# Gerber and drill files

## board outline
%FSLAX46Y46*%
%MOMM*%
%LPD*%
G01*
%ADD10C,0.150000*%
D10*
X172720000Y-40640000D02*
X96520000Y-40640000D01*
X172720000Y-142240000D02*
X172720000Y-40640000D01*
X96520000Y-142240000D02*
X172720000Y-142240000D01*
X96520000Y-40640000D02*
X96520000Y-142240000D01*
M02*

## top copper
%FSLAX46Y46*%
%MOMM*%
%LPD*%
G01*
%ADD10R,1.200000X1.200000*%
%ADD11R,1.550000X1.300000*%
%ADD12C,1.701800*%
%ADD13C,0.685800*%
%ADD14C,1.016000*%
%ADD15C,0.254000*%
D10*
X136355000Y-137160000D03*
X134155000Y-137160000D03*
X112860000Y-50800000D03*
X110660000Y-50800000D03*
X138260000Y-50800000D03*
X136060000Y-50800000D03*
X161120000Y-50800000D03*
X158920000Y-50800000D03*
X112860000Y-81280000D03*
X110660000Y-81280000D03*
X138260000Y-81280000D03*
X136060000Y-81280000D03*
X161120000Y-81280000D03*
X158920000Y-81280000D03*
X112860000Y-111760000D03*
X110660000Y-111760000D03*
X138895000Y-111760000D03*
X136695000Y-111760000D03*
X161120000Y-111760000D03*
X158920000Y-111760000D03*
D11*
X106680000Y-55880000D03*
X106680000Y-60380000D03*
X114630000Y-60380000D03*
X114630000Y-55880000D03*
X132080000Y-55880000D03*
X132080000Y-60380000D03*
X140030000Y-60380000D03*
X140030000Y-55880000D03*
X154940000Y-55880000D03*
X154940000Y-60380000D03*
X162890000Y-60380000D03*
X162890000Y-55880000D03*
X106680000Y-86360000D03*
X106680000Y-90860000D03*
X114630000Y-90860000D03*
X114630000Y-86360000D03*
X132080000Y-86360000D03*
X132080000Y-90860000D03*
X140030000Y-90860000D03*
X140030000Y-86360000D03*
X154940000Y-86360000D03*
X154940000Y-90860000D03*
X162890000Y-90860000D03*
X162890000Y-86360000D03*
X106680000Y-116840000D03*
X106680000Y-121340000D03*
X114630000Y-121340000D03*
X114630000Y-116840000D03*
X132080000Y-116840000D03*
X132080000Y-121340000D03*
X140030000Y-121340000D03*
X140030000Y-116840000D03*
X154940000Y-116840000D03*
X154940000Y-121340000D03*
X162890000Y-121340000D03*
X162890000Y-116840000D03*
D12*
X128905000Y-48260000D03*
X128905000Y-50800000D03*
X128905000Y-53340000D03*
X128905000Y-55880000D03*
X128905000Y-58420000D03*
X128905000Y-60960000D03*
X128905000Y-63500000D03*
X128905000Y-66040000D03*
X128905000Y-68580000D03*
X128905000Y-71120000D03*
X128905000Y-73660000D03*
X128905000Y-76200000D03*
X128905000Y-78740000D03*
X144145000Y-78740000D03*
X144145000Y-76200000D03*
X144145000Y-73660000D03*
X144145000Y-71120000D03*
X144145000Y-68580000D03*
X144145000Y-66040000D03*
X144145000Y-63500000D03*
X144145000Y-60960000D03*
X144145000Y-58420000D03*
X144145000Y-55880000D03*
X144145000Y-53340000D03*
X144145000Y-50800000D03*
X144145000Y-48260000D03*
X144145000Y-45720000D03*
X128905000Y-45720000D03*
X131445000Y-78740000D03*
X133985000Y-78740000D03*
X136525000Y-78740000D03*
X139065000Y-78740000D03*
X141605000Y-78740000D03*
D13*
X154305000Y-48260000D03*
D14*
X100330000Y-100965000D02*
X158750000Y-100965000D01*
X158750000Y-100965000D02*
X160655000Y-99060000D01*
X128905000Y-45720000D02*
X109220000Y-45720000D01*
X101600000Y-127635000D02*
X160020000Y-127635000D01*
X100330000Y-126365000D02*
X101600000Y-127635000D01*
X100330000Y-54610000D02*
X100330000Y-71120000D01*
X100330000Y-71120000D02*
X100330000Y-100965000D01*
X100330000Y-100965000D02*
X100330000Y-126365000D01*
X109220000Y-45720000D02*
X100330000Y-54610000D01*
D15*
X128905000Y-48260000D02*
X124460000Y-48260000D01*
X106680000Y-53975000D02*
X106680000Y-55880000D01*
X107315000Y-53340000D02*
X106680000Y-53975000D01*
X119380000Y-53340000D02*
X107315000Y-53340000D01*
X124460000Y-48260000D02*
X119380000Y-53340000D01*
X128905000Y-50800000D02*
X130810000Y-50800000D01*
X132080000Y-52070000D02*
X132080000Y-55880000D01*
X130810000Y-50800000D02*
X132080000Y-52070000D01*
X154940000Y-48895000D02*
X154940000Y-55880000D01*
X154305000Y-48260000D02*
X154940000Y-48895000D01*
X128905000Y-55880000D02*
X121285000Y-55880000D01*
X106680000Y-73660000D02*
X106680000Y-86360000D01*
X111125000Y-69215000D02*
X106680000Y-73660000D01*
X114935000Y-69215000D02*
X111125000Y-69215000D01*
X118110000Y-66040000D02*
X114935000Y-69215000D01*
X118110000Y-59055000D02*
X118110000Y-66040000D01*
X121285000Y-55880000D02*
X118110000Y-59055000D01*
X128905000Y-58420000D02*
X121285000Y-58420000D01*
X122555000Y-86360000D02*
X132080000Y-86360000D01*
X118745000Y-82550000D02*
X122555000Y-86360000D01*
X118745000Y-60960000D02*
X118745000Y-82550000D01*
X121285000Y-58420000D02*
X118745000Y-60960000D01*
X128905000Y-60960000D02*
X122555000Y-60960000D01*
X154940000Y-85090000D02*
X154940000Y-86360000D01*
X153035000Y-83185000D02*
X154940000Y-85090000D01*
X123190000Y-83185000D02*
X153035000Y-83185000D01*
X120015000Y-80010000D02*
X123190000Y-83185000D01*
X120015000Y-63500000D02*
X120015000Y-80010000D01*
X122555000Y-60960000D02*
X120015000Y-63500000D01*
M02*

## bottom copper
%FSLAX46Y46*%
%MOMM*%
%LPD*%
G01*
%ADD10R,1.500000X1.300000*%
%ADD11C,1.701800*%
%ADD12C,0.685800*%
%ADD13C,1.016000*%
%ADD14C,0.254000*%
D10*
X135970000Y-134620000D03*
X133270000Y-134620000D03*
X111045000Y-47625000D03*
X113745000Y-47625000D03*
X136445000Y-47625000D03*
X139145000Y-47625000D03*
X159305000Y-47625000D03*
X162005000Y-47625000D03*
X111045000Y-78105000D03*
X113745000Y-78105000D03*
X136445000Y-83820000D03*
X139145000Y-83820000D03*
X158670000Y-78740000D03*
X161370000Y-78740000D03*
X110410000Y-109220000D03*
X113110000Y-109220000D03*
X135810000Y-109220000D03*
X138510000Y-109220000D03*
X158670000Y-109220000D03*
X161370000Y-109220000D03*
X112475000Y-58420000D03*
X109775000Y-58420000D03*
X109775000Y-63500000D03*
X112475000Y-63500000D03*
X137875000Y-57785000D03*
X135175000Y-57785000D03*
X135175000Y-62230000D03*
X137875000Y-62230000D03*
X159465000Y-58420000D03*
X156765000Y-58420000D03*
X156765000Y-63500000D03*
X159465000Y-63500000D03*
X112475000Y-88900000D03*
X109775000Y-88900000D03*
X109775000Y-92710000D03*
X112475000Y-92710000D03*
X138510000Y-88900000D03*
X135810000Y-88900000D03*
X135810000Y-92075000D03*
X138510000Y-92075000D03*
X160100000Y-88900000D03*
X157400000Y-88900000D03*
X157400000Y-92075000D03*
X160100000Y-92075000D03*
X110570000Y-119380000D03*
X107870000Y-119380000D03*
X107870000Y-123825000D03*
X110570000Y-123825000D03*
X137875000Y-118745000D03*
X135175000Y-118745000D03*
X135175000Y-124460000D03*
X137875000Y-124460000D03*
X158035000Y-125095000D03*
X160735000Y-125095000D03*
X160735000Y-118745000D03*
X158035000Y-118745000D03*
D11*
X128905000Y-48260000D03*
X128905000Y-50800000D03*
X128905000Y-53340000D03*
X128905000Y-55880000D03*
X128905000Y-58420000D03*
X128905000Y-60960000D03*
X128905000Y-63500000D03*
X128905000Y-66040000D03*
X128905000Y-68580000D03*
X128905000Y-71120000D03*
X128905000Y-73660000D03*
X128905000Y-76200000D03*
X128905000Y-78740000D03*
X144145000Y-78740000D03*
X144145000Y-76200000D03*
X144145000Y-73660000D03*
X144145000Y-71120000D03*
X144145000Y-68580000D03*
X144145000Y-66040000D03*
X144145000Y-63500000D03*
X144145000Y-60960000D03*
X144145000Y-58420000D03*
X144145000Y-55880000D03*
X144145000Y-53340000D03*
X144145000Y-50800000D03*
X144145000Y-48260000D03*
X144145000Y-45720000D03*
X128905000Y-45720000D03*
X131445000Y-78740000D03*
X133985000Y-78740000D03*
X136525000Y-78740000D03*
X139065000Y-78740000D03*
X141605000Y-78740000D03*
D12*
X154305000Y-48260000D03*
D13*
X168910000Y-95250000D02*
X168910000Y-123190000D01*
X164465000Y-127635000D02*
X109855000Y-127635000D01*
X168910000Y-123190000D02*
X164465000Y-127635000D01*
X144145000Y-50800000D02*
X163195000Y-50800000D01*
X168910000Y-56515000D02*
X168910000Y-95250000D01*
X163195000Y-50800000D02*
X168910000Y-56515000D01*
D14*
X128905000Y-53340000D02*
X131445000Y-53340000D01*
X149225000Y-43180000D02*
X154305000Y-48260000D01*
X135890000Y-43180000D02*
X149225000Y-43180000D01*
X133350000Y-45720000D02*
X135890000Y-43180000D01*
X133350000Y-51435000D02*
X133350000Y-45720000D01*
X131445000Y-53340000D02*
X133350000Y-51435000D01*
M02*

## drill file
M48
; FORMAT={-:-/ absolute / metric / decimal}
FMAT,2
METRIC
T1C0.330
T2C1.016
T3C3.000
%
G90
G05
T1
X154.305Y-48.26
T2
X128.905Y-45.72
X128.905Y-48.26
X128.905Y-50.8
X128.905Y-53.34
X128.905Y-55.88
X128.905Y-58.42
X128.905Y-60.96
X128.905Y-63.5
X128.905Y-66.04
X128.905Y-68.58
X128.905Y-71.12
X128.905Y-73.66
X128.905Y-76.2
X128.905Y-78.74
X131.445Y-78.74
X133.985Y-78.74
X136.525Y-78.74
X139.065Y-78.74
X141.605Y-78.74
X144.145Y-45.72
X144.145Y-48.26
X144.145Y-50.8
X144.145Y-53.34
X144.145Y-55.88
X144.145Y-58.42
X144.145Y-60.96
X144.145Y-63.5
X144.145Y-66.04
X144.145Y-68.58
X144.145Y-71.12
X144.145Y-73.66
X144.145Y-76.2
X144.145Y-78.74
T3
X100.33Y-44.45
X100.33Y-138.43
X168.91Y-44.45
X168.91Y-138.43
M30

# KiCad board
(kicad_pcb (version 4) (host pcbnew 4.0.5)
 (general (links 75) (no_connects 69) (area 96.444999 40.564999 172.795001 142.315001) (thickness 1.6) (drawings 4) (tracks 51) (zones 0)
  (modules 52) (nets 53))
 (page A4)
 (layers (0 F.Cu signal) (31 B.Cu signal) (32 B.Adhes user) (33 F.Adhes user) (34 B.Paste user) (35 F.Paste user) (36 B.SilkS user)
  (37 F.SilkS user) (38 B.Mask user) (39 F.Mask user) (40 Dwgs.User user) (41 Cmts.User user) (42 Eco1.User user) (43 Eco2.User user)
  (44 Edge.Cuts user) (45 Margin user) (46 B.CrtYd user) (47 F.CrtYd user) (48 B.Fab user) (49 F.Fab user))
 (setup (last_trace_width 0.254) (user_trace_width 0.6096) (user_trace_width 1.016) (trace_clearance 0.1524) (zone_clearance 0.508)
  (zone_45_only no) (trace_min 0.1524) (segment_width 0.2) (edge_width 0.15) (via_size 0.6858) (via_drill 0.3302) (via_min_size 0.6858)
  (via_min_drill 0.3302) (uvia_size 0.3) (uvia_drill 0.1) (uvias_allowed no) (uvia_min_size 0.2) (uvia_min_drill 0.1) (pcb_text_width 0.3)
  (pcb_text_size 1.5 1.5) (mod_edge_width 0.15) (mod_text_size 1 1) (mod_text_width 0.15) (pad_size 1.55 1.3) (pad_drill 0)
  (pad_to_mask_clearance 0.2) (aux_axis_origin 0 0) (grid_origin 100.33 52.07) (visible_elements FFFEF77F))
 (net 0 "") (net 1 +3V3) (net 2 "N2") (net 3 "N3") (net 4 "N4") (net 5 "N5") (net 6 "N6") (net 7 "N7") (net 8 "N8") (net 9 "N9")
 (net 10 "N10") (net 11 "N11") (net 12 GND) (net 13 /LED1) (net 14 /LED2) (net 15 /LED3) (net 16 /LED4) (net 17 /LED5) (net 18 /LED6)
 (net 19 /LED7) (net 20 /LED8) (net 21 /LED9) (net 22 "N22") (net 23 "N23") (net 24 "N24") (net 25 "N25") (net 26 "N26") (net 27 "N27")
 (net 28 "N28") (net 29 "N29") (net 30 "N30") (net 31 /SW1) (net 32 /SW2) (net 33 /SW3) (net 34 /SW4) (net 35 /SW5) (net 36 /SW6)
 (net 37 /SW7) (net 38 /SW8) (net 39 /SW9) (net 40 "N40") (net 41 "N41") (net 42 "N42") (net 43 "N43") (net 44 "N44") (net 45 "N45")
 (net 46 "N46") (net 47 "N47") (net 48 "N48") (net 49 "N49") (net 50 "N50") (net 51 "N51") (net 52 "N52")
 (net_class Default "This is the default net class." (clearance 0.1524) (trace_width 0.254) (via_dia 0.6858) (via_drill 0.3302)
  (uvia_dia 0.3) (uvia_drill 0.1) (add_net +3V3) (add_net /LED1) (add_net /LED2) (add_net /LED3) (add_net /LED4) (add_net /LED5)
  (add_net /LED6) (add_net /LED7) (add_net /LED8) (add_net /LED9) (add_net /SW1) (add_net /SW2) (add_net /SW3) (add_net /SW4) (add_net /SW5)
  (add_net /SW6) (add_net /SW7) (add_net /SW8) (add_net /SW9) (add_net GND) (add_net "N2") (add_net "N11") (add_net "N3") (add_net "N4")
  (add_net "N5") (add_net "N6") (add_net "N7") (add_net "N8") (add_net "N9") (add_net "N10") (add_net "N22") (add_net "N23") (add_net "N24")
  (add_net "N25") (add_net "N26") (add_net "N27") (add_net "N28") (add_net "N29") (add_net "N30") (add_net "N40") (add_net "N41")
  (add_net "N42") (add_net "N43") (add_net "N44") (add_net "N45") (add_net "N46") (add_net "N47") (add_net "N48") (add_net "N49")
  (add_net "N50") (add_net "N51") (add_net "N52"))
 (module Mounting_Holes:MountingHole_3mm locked (layer F.Cu) (at 168.91 138.43)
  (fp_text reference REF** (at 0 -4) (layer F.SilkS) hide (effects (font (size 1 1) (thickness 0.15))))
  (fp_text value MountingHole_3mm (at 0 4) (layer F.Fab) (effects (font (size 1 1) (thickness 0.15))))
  (pad 1 np_thru_hole circle (at 0 0) (size 3 3) (drill 3) (layers *.Cu *.Mask)))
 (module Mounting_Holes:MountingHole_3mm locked (layer F.Cu) (at 100.33 138.43)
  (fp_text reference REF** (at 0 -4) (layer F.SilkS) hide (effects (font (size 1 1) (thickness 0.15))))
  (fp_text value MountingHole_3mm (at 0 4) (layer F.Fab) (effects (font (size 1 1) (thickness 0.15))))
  (pad 1 np_thru_hole circle (at 0 0) (size 3 3) (drill 3) (layers *.Cu *.Mask)))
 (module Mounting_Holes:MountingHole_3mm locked (layer F.Cu) (at 100.33 44.45)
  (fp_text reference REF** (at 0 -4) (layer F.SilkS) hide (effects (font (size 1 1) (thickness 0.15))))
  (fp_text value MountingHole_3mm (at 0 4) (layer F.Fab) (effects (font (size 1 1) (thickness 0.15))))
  (pad 1 np_thru_hole circle (at 0 0) (size 3 3) (drill 3) (layers *.Cu *.Mask)))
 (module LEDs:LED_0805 (layer F.Cu) (at 135.255 137.16)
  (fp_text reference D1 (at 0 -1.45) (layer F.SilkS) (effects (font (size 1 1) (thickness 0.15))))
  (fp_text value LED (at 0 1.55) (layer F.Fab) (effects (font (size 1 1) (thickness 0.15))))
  (pad 2 smd rect (at 1.1 0 180) (size 1.2 1.2) (layers F.Cu F.Paste F.Mask) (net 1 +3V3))
  (pad 1 smd rect (at -1.1 0 180) (size 1.2 1.2) (layers F.Cu F.Paste F.Mask) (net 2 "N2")))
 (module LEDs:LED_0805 (layer F.Cu) (at 111.76 50.8)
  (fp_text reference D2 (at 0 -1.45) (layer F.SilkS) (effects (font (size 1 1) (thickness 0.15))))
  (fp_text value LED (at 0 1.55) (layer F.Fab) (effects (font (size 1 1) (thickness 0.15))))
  (pad 2 smd rect (at 1.1 0 180) (size 1.2 1.2) (layers F.Cu F.Paste F.Mask) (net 1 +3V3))
  (pad 1 smd rect (at -1.1 0 180) (size 1.2 1.2) (layers F.Cu F.Paste F.Mask) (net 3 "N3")))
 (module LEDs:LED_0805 (layer F.Cu) (at 137.16 50.8)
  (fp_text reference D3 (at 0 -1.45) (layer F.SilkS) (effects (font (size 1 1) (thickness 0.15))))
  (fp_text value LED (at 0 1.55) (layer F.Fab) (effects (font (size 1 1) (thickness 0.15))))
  (pad 2 smd rect (at 1.1 0 180) (size 1.2 1.2) (layers F.Cu F.Paste F.Mask) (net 1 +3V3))
  (pad 1 smd rect (at -1.1 0 180) (size 1.2 1.2) (layers F.Cu F.Paste F.Mask) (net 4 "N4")))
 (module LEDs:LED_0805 (layer F.Cu) (at 160.02 50.8)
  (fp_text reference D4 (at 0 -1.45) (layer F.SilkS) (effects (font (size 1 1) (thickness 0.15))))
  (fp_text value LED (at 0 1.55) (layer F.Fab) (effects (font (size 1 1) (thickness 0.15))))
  (pad 2 smd rect (at 1.1 0 180) (size 1.2 1.2) (layers F.Cu F.Paste F.Mask) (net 1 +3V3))
  (pad 1 smd rect (at -1.1 0 180) (size 1.2 1.2) (layers F.Cu F.Paste F.Mask) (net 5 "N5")))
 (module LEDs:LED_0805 (layer F.Cu) (at 111.76 81.28)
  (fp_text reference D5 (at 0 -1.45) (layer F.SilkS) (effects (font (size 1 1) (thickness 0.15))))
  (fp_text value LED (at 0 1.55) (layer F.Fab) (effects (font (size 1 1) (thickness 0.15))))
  (pad 2 smd rect (at 1.1 0 180) (size 1.2 1.2) (layers F.Cu F.Paste F.Mask) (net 1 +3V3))
  (pad 1 smd rect (at -1.1 0 180) (size 1.2 1.2) (layers F.Cu F.Paste F.Mask) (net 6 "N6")))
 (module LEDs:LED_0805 (layer F.Cu) (at 137.16 81.28)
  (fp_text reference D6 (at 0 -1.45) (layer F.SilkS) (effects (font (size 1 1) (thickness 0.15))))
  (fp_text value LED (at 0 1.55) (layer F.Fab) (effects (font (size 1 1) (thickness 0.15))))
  (pad 2 smd rect (at 1.1 0 180) (size 1.2 1.2) (layers F.Cu F.Paste F.Mask) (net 1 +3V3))
  (pad 1 smd rect (at -1.1 0 180) (size 1.2 1.2) (layers F.Cu F.Paste F.Mask) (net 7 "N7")))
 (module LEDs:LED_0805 (layer F.Cu) (at 160.02 81.28)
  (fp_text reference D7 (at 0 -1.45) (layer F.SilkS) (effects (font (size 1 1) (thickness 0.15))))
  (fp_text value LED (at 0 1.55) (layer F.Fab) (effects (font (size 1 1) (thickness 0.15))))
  (pad 2 smd rect (at 1.1 0 180) (size 1.2 1.2) (layers F.Cu F.Paste F.Mask) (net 1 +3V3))
  (pad 1 smd rect (at -1.1 0 180) (size 1.2 1.2) (layers F.Cu F.Paste F.Mask) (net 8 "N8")))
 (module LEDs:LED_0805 (layer F.Cu) (at 111.76 111.76)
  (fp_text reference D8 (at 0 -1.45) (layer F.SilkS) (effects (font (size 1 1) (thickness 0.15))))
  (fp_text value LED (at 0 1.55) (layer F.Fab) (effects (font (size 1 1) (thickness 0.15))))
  (pad 2 smd rect (at 1.1 0 180) (size 1.2 1.2) (layers F.Cu F.Paste F.Mask) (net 1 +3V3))
  (pad 1 smd rect (at -1.1 0 180) (size 1.2 1.2) (layers F.Cu F.Paste F.Mask) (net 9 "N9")))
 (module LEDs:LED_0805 (layer F.Cu) (at 137.795 111.76)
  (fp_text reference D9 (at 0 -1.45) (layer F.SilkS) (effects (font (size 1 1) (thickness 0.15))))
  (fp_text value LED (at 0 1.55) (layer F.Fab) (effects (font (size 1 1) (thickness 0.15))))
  (pad 2 smd rect (at 1.1 0 180) (size 1.2 1.2) (layers F.Cu F.Paste F.Mask) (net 1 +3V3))
  (pad 1 smd rect (at -1.1 0 180) (size 1.2 1.2) (layers F.Cu F.Paste F.Mask) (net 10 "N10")))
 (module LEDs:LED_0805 (layer F.Cu) (at 160.02 111.76)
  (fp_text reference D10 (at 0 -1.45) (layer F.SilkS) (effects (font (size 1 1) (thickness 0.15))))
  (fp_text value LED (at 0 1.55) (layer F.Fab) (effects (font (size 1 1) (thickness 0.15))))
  (pad 2 smd rect (at 1.1 0 180) (size 1.2 1.2) (layers F.Cu F.Paste F.Mask) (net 1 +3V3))
  (pad 1 smd rect (at -1.1 0 180) (size 1.2 1.2) (layers F.Cu F.Paste F.Mask) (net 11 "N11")))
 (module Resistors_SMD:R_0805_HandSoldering (layer B.Cu) (at 134.62 134.62 180)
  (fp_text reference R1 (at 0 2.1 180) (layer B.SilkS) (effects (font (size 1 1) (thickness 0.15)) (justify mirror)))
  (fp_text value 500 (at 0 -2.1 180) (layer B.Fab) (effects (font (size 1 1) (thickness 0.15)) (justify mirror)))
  (pad 1 smd rect (at -1.35 0 180) (size 1.5 1.3) (layers B.Cu B.Paste B.Mask) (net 2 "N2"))
  (pad 2 smd rect (at 1.35 0 180) (size 1.5 1.3) (layers B.Cu B.Paste B.Mask) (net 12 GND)))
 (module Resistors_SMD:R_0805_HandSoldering (layer B.Cu) (at 112.395 47.625)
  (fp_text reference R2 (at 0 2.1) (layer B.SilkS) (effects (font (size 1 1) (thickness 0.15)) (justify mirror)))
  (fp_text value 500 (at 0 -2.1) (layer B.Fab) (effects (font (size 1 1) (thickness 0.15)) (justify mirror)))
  (pad 1 smd rect (at -1.35 0) (size 1.5 1.3) (layers B.Cu B.Paste B.Mask) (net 3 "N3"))
  (pad 2 smd rect (at 1.35 0) (size 1.5 1.3) (layers B.Cu B.Paste B.Mask) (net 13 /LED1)))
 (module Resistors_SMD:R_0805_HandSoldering (layer B.Cu) (at 137.795 47.625)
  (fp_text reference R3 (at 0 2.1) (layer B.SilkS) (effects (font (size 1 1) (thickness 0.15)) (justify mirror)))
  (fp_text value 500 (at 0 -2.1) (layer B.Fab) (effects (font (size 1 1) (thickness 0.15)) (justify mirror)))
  (pad 1 smd rect (at -1.35 0) (size 1.5 1.3) (layers B.Cu B.Paste B.Mask) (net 4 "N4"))
  (pad 2 smd rect (at 1.35 0) (size 1.5 1.3) (layers B.Cu B.Paste B.Mask) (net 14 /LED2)))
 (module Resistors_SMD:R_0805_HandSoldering (layer B.Cu) (at 160.655 47.625)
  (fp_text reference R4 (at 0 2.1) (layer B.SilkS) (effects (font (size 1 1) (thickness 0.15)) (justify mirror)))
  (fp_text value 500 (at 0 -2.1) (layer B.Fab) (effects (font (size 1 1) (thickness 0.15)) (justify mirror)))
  (pad 1 smd rect (at -1.35 0) (size 1.5 1.3) (layers B.Cu B.Paste B.Mask) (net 5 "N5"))
  (pad 2 smd rect (at 1.35 0) (size 1.5 1.3) (layers B.Cu B.Paste B.Mask) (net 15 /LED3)))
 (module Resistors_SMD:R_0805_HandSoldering (layer B.Cu) (at 112.395 78.105)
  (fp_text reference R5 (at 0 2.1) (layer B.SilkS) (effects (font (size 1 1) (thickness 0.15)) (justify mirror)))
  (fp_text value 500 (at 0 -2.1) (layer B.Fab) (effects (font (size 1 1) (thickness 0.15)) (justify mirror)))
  (pad 1 smd rect (at -1.35 0) (size 1.5 1.3) (layers B.Cu B.Paste B.Mask) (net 6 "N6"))
  (pad 2 smd rect (at 1.35 0) (size 1.5 1.3) (layers B.Cu B.Paste B.Mask) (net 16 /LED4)))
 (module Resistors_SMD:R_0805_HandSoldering (layer B.Cu) (at 137.795 83.82)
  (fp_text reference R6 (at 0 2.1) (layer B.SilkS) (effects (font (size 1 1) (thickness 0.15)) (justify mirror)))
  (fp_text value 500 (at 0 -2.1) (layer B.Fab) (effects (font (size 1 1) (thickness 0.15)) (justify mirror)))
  (pad 1 smd rect (at -1.35 0) (size 1.5 1.3) (layers B.Cu B.Paste B.Mask) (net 7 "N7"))
  (pad 2 smd rect (at 1.35 0) (size 1.5 1.3) (layers B.Cu B.Paste B.Mask) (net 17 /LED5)))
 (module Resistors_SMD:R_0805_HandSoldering (layer B.Cu) (at 160.02 78.74)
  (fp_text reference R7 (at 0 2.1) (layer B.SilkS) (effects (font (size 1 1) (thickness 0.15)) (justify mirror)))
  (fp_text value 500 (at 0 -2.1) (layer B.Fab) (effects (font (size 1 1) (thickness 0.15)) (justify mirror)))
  (pad 1 smd rect (at -1.35 0) (size 1.5 1.3) (layers B.Cu B.Paste B.Mask) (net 8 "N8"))
  (pad 2 smd rect (at 1.35 0) (size 1.5 1.3) (layers B.Cu B.Paste B.Mask) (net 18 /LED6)))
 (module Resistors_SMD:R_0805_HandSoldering (layer B.Cu) (at 111.76 109.22)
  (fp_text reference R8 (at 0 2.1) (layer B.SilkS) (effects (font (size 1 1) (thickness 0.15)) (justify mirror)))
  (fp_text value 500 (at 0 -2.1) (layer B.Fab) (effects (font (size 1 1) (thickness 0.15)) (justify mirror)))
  (pad 1 smd rect (at -1.35 0) (size 1.5 1.3) (layers B.Cu B.Paste B.Mask) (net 9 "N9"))
  (pad 2 smd rect (at 1.35 0) (size 1.5 1.3) (layers B.Cu B.Paste B.Mask) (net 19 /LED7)))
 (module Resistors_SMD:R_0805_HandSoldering (layer B.Cu) (at 137.16 109.22)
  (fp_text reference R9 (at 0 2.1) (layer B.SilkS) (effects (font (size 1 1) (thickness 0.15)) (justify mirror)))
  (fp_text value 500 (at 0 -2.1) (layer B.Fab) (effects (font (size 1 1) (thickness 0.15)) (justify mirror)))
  (pad 1 smd rect (at -1.35 0) (size 1.5 1.3) (layers B.Cu B.Paste B.Mask) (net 10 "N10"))
  (pad 2 smd rect (at 1.35 0) (size 1.5 1.3) (layers B.Cu B.Paste B.Mask) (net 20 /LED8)))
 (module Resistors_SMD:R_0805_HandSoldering (layer B.Cu) (at 160.02 109.22)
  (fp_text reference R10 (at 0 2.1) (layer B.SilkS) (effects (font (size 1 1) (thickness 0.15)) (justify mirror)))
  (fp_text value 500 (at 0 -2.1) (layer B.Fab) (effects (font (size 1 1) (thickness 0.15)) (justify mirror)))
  (pad 1 smd rect (at -1.35 0) (size 1.5 1.3) (layers B.Cu B.Paste B.Mask) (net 11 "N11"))
  (pad 2 smd rect (at 1.35 0) (size 1.5 1.3) (layers B.Cu B.Paste B.Mask) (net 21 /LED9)))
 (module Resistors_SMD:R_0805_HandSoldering (layer B.Cu) (at 111.125 58.42 180)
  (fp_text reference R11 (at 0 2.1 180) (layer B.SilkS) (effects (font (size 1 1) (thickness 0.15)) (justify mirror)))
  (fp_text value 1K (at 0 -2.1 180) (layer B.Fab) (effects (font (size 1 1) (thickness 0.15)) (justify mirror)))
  (pad 1 smd rect (at -1.35 0 180) (size 1.5 1.3) (layers B.Cu B.Paste B.Mask) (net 1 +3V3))
  (pad 2 smd rect (at 1.35 0 180) (size 1.5 1.3) (layers B.Cu B.Paste B.Mask) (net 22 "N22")))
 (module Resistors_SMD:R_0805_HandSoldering (layer B.Cu) (at 111.125 63.5)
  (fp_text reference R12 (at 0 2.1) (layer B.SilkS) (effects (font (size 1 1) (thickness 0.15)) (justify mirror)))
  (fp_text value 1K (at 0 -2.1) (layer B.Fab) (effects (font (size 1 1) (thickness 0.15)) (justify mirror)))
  (pad 1 smd rect (at -1.35 0) (size 1.5 1.3) (layers B.Cu B.Paste B.Mask) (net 22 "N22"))
  (pad 2 smd rect (at 1.35 0) (size 1.5 1.3) (layers B.Cu B.Paste B.Mask) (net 12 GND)))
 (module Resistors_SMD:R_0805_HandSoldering (layer B.Cu) (at 136.525 57.785 180)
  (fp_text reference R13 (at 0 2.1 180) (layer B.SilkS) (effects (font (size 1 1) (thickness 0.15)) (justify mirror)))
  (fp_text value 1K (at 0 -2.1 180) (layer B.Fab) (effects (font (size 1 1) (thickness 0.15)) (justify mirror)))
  (pad 1 smd rect (at -1.35 0 180) (size 1.5 1.3) (layers B.Cu B.Paste B.Mask) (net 1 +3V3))
  (pad 2 smd rect (at 1.35 0 180) (size 1.5 1.3) (layers B.Cu B.Paste B.Mask) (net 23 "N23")))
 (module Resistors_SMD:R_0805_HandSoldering (layer B.Cu) (at 136.525 62.23)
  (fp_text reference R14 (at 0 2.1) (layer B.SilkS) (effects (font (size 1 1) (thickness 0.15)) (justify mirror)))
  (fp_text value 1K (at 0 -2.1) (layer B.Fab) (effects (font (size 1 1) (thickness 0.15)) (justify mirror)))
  (pad 1 smd rect (at -1.35 0) (size 1.5 1.3) (layers B.Cu B.Paste B.Mask) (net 23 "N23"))
  (pad 2 smd rect (at 1.35 0) (size 1.5 1.3) (layers B.Cu B.Paste B.Mask) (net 12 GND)))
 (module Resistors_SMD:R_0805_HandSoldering (layer B.Cu) (at 158.115 58.42 180)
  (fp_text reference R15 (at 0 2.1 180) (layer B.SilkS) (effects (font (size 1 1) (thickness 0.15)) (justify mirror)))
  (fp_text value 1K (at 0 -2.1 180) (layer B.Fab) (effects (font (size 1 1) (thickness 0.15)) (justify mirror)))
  (pad 1 smd rect (at -1.35 0 180) (size 1.5 1.3) (layers B.Cu B.Paste B.Mask) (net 1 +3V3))
  (pad 2 smd rect (at 1.35 0 180) (size 1.5 1.3) (layers B.Cu B.Paste B.Mask) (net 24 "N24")))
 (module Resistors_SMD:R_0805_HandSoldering (layer B.Cu) (at 158.115 63.5)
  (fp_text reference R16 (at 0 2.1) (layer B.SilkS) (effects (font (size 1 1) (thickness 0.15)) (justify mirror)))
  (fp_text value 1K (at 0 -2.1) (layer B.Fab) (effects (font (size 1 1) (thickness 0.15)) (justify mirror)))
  (pad 1 smd rect (at -1.35 0) (size 1.5 1.3) (layers B.Cu B.Paste B.Mask) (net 24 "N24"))
  (pad 2 smd rect (at 1.35 0) (size 1.5 1.3) (layers B.Cu B.Paste B.Mask) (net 12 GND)))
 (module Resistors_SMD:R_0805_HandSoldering (layer B.Cu) (at 111.125 88.9 180)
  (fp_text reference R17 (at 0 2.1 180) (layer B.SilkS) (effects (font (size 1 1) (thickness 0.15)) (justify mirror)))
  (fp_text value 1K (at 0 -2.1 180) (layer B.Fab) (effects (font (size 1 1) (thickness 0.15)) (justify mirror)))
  (pad 1 smd rect (at -1.35 0 180) (size 1.5 1.3) (layers B.Cu B.Paste B.Mask) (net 1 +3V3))
  (pad 2 smd rect (at 1.35 0 180) (size 1.5 1.3) (layers B.Cu B.Paste B.Mask) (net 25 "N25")))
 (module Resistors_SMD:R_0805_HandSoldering (layer B.Cu) (at 111.125 92.71)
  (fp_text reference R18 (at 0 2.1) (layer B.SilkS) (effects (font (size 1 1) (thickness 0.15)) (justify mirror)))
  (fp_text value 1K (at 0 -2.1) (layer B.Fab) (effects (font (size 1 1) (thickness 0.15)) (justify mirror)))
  (pad 1 smd rect (at -1.35 0) (size 1.5 1.3) (layers B.Cu B.Paste B.Mask) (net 25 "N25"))
  (pad 2 smd rect (at 1.35 0) (size 1.5 1.3) (layers B.Cu B.Paste B.Mask) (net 12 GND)))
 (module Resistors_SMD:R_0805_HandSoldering (layer B.Cu) (at 137.16 88.9 180)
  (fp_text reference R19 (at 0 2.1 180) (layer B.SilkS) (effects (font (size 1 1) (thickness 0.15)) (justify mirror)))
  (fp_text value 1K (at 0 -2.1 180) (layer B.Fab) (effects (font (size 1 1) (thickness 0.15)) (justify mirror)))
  (pad 1 smd rect (at -1.35 0 180) (size 1.5 1.3) (layers B.Cu B.Paste B.Mask) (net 1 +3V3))
  (pad 2 smd rect (at 1.35 0 180) (size 1.5 1.3) (layers B.Cu B.Paste B.Mask) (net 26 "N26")))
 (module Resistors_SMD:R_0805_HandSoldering (layer B.Cu) (at 137.16 92.075)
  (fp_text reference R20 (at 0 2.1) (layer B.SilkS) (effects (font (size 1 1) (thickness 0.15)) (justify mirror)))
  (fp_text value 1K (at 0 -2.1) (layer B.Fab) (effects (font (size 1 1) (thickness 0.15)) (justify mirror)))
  (pad 1 smd rect (at -1.35 0) (size 1.5 1.3) (layers B.Cu B.Paste B.Mask) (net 26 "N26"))
  (pad 2 smd rect (at 1.35 0) (size 1.5 1.3) (layers B.Cu B.Paste B.Mask) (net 12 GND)))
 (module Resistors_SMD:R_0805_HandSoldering (layer B.Cu) (at 158.75 88.9 180)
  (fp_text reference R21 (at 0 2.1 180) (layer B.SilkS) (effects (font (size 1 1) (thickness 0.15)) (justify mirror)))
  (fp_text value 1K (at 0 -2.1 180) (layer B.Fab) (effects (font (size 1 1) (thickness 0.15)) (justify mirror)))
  (pad 1 smd rect (at -1.35 0 180) (size 1.5 1.3) (layers B.Cu B.Paste B.Mask) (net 1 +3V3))
  (pad 2 smd rect (at 1.35 0 180) (size 1.5 1.3) (layers B.Cu B.Paste B.Mask) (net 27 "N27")))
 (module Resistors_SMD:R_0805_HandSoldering (layer B.Cu) (at 158.75 92.075)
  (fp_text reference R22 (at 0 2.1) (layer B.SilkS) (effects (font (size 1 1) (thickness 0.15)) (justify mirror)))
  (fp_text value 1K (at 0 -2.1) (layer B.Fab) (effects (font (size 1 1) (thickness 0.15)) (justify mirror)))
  (pad 1 smd rect (at -1.35 0) (size 1.5 1.3) (layers B.Cu B.Paste B.Mask) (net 27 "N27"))
  (pad 2 smd rect (at 1.35 0) (size 1.5 1.3) (layers B.Cu B.Paste B.Mask) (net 12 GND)))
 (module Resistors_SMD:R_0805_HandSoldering (layer B.Cu) (at 109.22 119.38 180)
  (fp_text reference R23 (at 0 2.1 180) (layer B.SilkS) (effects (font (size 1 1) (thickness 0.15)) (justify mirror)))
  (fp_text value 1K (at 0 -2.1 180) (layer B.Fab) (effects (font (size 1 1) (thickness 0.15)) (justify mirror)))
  (pad 1 smd rect (at -1.35 0 180) (size 1.5 1.3) (layers B.Cu B.Paste B.Mask) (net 1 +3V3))
  (pad 2 smd rect (at 1.35 0 180) (size 1.5 1.3) (layers B.Cu B.Paste B.Mask) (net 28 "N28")))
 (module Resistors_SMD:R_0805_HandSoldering (layer B.Cu) (at 109.22 123.825)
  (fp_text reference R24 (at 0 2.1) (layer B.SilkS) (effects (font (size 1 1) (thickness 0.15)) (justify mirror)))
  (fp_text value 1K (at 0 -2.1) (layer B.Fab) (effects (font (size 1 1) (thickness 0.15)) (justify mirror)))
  (pad 1 smd rect (at -1.35 0) (size 1.5 1.3) (layers B.Cu B.Paste B.Mask) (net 28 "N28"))
  (pad 2 smd rect (at 1.35 0) (size 1.5 1.3) (layers B.Cu B.Paste B.Mask) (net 12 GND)))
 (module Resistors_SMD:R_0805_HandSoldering (layer B.Cu) (at 136.525 118.745 180)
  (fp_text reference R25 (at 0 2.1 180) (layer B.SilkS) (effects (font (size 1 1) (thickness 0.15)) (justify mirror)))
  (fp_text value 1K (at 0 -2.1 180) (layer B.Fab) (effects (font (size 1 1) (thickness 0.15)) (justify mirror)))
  (pad 1 smd rect (at -1.35 0 180) (size 1.5 1.3) (layers B.Cu B.Paste B.Mask) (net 1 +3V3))
  (pad 2 smd rect (at 1.35 0 180) (size 1.5 1.3) (layers B.Cu B.Paste B.Mask) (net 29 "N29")))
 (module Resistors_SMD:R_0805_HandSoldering (layer B.Cu) (at 136.525 124.46)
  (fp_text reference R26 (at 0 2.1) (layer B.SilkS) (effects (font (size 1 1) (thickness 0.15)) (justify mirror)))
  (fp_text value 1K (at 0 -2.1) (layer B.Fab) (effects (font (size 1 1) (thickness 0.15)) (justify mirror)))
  (pad 1 smd rect (at -1.35 0) (size 1.5 1.3) (layers B.Cu B.Paste B.Mask) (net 29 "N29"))
  (pad 2 smd rect (at 1.35 0) (size 1.5 1.3) (layers B.Cu B.Paste B.Mask) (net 12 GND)))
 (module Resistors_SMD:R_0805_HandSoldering (layer B.Cu) (at 159.385 125.095)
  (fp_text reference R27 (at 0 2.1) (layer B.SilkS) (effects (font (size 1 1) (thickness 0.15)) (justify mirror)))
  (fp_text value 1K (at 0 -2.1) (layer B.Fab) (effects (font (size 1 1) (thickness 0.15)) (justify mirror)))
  (pad 1 smd rect (at -1.35 0) (size 1.5 1.3) (layers B.Cu B.Paste B.Mask) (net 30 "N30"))
  (pad 2 smd rect (at 1.35 0) (size 1.5 1.3) (layers B.Cu B.Paste B.Mask) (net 12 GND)))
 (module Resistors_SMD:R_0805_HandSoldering (layer B.Cu) (at 159.385 118.745 180)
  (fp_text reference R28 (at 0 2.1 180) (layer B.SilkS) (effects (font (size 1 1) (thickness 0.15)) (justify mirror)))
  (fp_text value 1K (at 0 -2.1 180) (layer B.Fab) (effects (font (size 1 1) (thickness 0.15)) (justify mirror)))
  (pad 1 smd rect (at -1.35 0 180) (size 1.5 1.3) (layers B.Cu B.Paste B.Mask) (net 1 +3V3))
  (pad 2 smd rect (at 1.35 0 180) (size 1.5 1.3) (layers B.Cu B.Paste B.Mask) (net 30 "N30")))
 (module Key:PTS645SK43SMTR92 (layer F.Cu) (at 106.68 55.88)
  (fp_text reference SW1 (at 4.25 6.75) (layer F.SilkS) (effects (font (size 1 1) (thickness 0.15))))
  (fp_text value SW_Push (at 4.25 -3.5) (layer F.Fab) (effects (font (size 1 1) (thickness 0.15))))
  (pad 1 smd rect (at 0 0) (size 1.55 1.3) (layers F.Cu F.Paste F.Mask) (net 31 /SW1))
  (pad 2 smd rect (at 0 4.5) (size 1.55 1.3) (layers F.Cu F.Paste F.Mask) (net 22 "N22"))
  (pad 3 smd rect (at 7.95 4.5) (size 1.55 1.3) (layers F.Cu F.Paste F.Mask))
  (pad 4 smd rect (at 7.95 0) (size 1.55 1.3) (layers F.Cu F.Paste F.Mask)))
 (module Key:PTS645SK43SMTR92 (layer F.Cu) (at 132.08 55.88)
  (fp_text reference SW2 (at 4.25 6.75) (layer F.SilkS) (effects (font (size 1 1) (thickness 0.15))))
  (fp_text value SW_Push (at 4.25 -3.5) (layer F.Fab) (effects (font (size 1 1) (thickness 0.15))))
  (pad 1 smd rect (at 0 0) (size 1.55 1.3) (layers F.Cu F.Paste F.Mask) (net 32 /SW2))
  (pad 2 smd rect (at 0 4.5) (size 1.55 1.3) (layers F.Cu F.Paste F.Mask) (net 23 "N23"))
  (pad 3 smd rect (at 7.95 4.5) (size 1.55 1.3) (layers F.Cu F.Paste F.Mask))
  (pad 4 smd rect (at 7.95 0) (size 1.55 1.3) (layers F.Cu F.Paste F.Mask)))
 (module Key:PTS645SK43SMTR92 (layer F.Cu) (at 154.94 55.88)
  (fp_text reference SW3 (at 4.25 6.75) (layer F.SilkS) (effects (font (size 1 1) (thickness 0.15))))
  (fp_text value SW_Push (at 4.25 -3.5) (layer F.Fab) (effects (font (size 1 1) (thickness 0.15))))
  (pad 1 smd rect (at 0 0) (size 1.55 1.3) (layers F.Cu F.Paste F.Mask) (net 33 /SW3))
  (pad 2 smd rect (at 0 4.5) (size 1.55 1.3) (layers F.Cu F.Paste F.Mask) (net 24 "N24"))
  (pad 3 smd rect (at 7.95 4.5) (size 1.55 1.3) (layers F.Cu F.Paste F.Mask))
  (pad 4 smd rect (at 7.95 0) (size 1.55 1.3) (layers F.Cu F.Paste F.Mask)))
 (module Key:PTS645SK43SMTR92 (layer F.Cu) (at 106.68 86.36)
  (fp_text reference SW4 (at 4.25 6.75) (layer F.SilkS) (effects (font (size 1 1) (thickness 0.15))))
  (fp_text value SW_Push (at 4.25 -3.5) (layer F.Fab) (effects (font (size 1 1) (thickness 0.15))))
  (pad 1 smd rect (at 0 0) (size 1.55 1.3) (layers F.Cu F.Paste F.Mask) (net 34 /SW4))
  (pad 2 smd rect (at 0 4.5) (size 1.55 1.3) (layers F.Cu F.Paste F.Mask) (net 25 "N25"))
  (pad 3 smd rect (at 7.95 4.5) (size 1.55 1.3) (layers F.Cu F.Paste F.Mask))
  (pad 4 smd rect (at 7.95 0) (size 1.55 1.3) (layers F.Cu F.Paste F.Mask)))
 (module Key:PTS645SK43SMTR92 (layer F.Cu) (at 132.08 86.36)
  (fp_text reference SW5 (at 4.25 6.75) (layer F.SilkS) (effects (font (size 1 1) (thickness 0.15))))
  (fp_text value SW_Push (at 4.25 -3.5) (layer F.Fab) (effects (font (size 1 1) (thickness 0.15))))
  (pad 1 smd rect (at 0 0) (size 1.55 1.3) (layers F.Cu F.Paste F.Mask) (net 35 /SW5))
  (pad 2 smd rect (at 0 4.5) (size 1.55 1.3) (layers F.Cu F.Paste F.Mask) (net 26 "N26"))
  (pad 3 smd rect (at 7.95 4.5) (size 1.55 1.3) (layers F.Cu F.Paste F.Mask))
  (pad 4 smd rect (at 7.95 0) (size 1.55 1.3) (layers F.Cu F.Paste F.Mask)))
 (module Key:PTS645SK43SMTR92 (layer F.Cu) (at 154.94 86.36)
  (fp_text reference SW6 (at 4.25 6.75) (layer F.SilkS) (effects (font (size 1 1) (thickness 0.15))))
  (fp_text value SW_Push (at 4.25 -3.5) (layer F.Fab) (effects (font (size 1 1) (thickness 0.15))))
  (pad 1 smd rect (at 0 0) (size 1.55 1.3) (layers F.Cu F.Paste F.Mask) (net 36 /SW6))
  (pad 2 smd rect (at 0 4.5) (size 1.55 1.3) (layers F.Cu F.Paste F.Mask) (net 27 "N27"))
  (pad 3 smd rect (at 7.95 4.5) (size 1.55 1.3) (layers F.Cu F.Paste F.Mask))
  (pad 4 smd rect (at 7.95 0) (size 1.55 1.3) (layers F.Cu F.Paste F.Mask)))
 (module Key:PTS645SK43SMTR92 (layer F.Cu) (at 106.68 116.84)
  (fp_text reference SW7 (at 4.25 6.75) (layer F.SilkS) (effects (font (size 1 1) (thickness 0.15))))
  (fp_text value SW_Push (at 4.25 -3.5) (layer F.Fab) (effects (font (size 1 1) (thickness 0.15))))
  (pad 1 smd rect (at 0 0) (size 1.55 1.3) (layers F.Cu F.Paste F.Mask) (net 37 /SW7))
  (pad 2 smd rect (at 0 4.5) (size 1.55 1.3) (layers F.Cu F.Paste F.Mask) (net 28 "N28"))
  (pad 3 smd rect (at 7.95 4.5) (size 1.55 1.3) (layers F.Cu F.Paste F.Mask))
  (pad 4 smd rect (at 7.95 0) (size 1.55 1.3) (layers F.Cu F.Paste F.Mask)))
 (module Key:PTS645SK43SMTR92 (layer F.Cu) (at 132.08 116.84)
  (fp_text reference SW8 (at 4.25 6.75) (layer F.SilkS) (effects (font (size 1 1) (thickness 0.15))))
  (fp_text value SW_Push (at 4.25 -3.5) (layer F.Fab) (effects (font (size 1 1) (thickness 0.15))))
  (pad 1 smd rect (at 0 0) (size 1.55 1.3) (layers F.Cu F.Paste F.Mask) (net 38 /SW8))
  (pad 2 smd rect (at 0 4.5) (size 1.55 1.3) (layers F.Cu F.Paste F.Mask) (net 29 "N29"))
  (pad 3 smd rect (at 7.95 4.5) (size 1.55 1.3) (layers F.Cu F.Paste F.Mask))
  (pad 4 smd rect (at 7.95 0) (size 1.55 1.3) (layers F.Cu F.Paste F.Mask)))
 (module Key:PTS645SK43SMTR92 (layer F.Cu) (at 154.94 116.84)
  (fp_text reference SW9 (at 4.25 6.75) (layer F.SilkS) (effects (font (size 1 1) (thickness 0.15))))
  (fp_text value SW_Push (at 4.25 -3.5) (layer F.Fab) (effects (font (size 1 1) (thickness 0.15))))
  (pad 1 smd rect (at 0 0) (size 1.55 1.3) (layers F.Cu F.Paste F.Mask) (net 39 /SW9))
  (pad 2 smd rect (at 0 4.5) (size 1.55 1.3) (layers F.Cu F.Paste F.Mask) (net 30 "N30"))
  (pad 3 smd rect (at 7.95 4.5) (size 1.55 1.3) (layers F.Cu F.Paste F.Mask))
  (pad 4 smd rect (at 7.95 0) (size 1.55 1.3) (layers F.Cu F.Paste F.Mask)))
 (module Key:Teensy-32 (layer B.Cu) (at 136.525 60.96 180)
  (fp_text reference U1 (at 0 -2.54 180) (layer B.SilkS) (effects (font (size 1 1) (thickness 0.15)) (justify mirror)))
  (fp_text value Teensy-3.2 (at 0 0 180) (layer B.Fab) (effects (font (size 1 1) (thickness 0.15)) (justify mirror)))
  (pad 0 thru_hole circle (at 7.62 12.7 180) (size 1.7018 1.7018) (drill 1.016) (layers *.Cu *.Mask) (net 31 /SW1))
  (pad 1 thru_hole circle (at 7.62 10.16 180) (size 1.7018 1.7018) (drill 1.016) (layers *.Cu *.Mask) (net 32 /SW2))
  (pad 2 thru_hole circle (at 7.62 7.62 180) (size 1.7018 1.7018) (drill 1.016) (layers *.Cu *.Mask) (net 33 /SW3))
  (pad 3 thru_hole circle (at 7.62 5.08 180) (size 1.7018 1.7018) (drill 1.016) (layers *.Cu *.Mask) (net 34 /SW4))
  (pad 4 thru_hole circle (at 7.62 2.54 180) (size 1.7018 1.7018) (drill 1.016) (layers *.Cu *.Mask) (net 35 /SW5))
  (pad 5 thru_hole circle (at 7.62 0 180) (size 1.7018 1.7018) (drill 1.016) (layers *.Cu *.Mask) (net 36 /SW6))
  (pad 6 thru_hole circle (at 7.62 -2.54 180) (size 1.7018 1.7018) (drill 1.016) (layers *.Cu *.Mask) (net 37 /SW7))
  (pad 7 thru_hole circle (at 7.62 -5.08 180) (size 1.7018 1.7018) (drill 1.016) (layers *.Cu *.Mask) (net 38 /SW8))
  (pad 8 thru_hole circle (at 7.62 -7.62 180) (size 1.7018 1.7018) (drill 1.016) (layers *.Cu *.Mask) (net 39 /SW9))
  (pad 9 thru_hole circle (at 7.62 -10.16 180) (size 1.7018 1.7018) (drill 1.016) (layers *.Cu *.Mask) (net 13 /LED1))
  (pad 10 thru_hole circle (at 7.62 -12.7 180) (size 1.7018 1.7018) (drill 1.016) (layers *.Cu *.Mask) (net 14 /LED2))
  (pad 11 thru_hole circle (at 7.62 -15.24 180) (size 1.7018 1.7018) (drill 1.016) (layers *.Cu *.Mask) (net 15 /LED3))
  (pad 12 thru_hole circle (at 7.62 -17.78 180) (size 1.7018 1.7018) (drill 1.016) (layers *.Cu *.Mask) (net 16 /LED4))
  (pad 13 thru_hole circle (at -7.62 -17.78 180) (size 1.7018 1.7018) (drill 1.016) (layers *.Cu *.Mask) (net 17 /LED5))
  (pad 14 thru_hole circle (at -7.62 -15.24 180) (size 1.7018 1.7018) (drill 1.016) (layers *.Cu *.Mask) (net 18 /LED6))
  (pad 15 thru_hole circle (at -7.62 -12.7 180) (size 1.7018 1.7018) (drill 1.016) (layers *.Cu *.Mask) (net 19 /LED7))
  (pad 16 thru_hole circle (at -7.62 -10.16 180) (size 1.7018 1.7018) (drill 1.016) (layers *.Cu *.Mask) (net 20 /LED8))
  (pad 17 thru_hole circle (at -7.62 -7.62 180) (size 1.7018 1.7018) (drill 1.016) (layers *.Cu *.Mask) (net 21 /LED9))
  (pad 18 thru_hole circle (at -7.62 -5.08 180) (size 1.7018 1.7018) (drill 1.016) (layers *.Cu *.Mask) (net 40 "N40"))
  (pad 19 thru_hole circle (at -7.62 -2.54 180) (size 1.7018 1.7018) (drill 1.016) (layers *.Cu *.Mask) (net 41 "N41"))
  (pad 20 thru_hole circle (at -7.62 0 180) (size 1.7018 1.7018) (drill 1.016) (layers *.Cu *.Mask) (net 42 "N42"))
  (pad 21 thru_hole circle (at -7.62 2.54 180) (size 1.7018 1.7018) (drill 1.016) (layers *.Cu *.Mask) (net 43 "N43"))
  (pad 22 thru_hole circle (at -7.62 5.08 180) (size 1.7018 1.7018) (drill 1.016) (layers *.Cu *.Mask) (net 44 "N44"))
  (pad 23 thru_hole circle (at -7.62 7.62 180) (size 1.7018 1.7018) (drill 1.016) (layers *.Cu *.Mask) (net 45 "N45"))
  (pad 24 thru_hole circle (at -7.62 10.16 180) (size 1.7018 1.7018) (drill 1.016) (layers *.Cu *.Mask) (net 1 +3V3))
  (pad 25 thru_hole circle (at -7.62 12.7 180) (size 1.7018 1.7018) (drill 1.016) (layers *.Cu *.Mask) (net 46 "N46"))
  (pad 26 thru_hole circle (at -7.62 15.24 180) (size 1.7018 1.7018) (drill 1.016) (layers *.Cu *.Mask) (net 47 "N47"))
  (pad 27 thru_hole circle (at 7.62 15.24 180) (size 1.7018 1.7018) (drill 1.016) (layers *.Cu *.Mask) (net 12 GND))
  (pad 28 thru_hole circle (at 5.08 -17.78 180) (size 1.7018 1.7018) (drill 1.016) (layers *.Cu *.Mask) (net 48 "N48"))
  (pad 29 thru_hole circle (at 2.54 -17.78 180) (size 1.7018 1.7018) (drill 1.016) (layers *.Cu *.Mask) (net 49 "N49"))
  (pad 30 thru_hole circle (at 0 -17.78 180) (size 1.7018 1.7018) (drill 1.016) (layers *.Cu *.Mask) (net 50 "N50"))
  (pad 31 thru_hole circle (at -2.54 -17.78 180) (size 1.7018 1.7018) (drill 1.016) (layers *.Cu *.Mask) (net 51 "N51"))
  (pad 32 thru_hole circle (at -5.08 -17.78 180) (size 1.7018 1.7018) (drill 1.016) (layers *.Cu *.Mask) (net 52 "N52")))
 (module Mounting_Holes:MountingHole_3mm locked (layer F.Cu) (at 168.91 44.45)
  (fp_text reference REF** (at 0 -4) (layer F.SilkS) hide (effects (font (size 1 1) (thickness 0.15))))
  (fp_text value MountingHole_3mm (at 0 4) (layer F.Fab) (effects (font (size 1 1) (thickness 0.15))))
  (pad 1 np_thru_hole circle (at 0 0) (size 3 3) (drill 3) (layers *.Cu *.Mask)))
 (gr_line (start 172.72 40.64) (end 96.52 40.64) (angle 90) (layer Edge.Cuts) (width 0.15))
 (gr_line (start 172.72 142.24) (end 172.72 40.64) (angle 90) (layer Edge.Cuts) (width 0.15))
 (gr_line (start 96.52 142.24) (end 172.72 142.24) (angle 90) (layer Edge.Cuts) (width 0.15))
 (gr_line (start 96.52 40.64) (end 96.52 142.24) (angle 90) (layer Edge.Cuts) (width 0.15))
 (segment (start 168.91 95.25) (end 168.91 123.19) (width 1.016) (layer B.Cu) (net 1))
 (segment (start 164.465 127.635) (end 109.855 127.635) (width 1.016) (layer B.Cu) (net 1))
 (segment (start 168.91 123.19) (end 164.465 127.635) (width 1.016) (layer B.Cu) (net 1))
 (segment (start 144.145 50.8) (end 163.195 50.8) (width 1.016) (layer B.Cu) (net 1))
 (segment (start 168.91 56.515) (end 168.91 95.25) (width 1.016) (layer B.Cu) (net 1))
 (segment (start 163.195 50.8) (end 168.91 56.515) (width 1.016) (layer B.Cu) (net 1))
 (segment (start 100.33 100.965) (end 158.75 100.965) (width 1.016) (layer F.Cu) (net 12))
 (segment (start 158.75 100.965) (end 160.655 99.06) (width 1.016) (layer F.Cu) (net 12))
 (segment (start 128.905 45.72) (end 109.22 45.72) (width 1.016) (layer F.Cu) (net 12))
 (segment (start 101.6 127.635) (end 160.02 127.635) (width 1.016) (layer F.Cu) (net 12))
 (segment (start 100.33 126.365) (end 101.6 127.635) (width 1.016) (layer F.Cu) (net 12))
 (segment (start 100.33 54.61) (end 100.33 71.12) (width 1.016) (layer F.Cu) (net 12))
 (segment (start 100.33 71.12) (end 100.33 100.965) (width 1.016) (layer F.Cu) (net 12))
 (segment (start 100.33 100.965) (end 100.33 126.365) (width 1.016) (layer F.Cu) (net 12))
 (segment (start 109.22 45.72) (end 100.33 54.61) (width 1.016) (layer F.Cu) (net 12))
 (segment (start 128.905 48.26) (end 124.46 48.26) (width 0.254) (layer F.Cu) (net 31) (status 400000))
 (segment (start 106.68 53.975) (end 106.68 55.88) (width 0.254) (layer F.Cu) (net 31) (status 800000))
 (segment (start 107.315 53.34) (end 106.68 53.975) (width 0.254) (layer F.Cu) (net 31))
 (segment (start 119.38 53.34) (end 107.315 53.34) (width 0.254) (layer F.Cu) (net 31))
 (segment (start 124.46 48.26) (end 119.38 53.34) (width 0.254) (layer F.Cu) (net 31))
 (segment (start 128.905 50.8) (end 130.81 50.8) (width 0.254) (layer F.Cu) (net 32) (status 400000))
 (segment (start 132.08 52.07) (end 132.08 55.88) (width 0.254) (layer F.Cu) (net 32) (status 800000))
 (segment (start 130.81 50.8) (end 132.08 52.07) (width 0.254) (layer F.Cu) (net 32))
 (segment (start 128.905 53.34) (end 131.445 53.34) (width 0.254) (layer B.Cu) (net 33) (status 400000))
 (segment (start 154.94 48.895) (end 154.94 55.88) (width 0.254) (layer F.Cu) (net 33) (status 800000))
 (segment (start 154.305 48.26) (end 154.94 48.895) (width 0.254) (layer F.Cu) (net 33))
 (via (at 154.305 48.26) (size 0.6858) (drill 0.3302) (layers F.Cu B.Cu) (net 33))
 (segment (start 149.225 43.18) (end 154.305 48.26) (width 0.254) (layer B.Cu) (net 33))
 (segment (start 135.89 43.18) (end 149.225 43.18) (width 0.254) (layer B.Cu) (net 33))
 (segment (start 133.35 45.72) (end 135.89 43.18) (width 0.254) (layer B.Cu) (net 33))
 (segment (start 133.35 51.435) (end 133.35 45.72) (width 0.254) (layer B.Cu) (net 33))
 (segment (start 131.445 53.34) (end 133.35 51.435) (width 0.254) (layer B.Cu) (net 33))
 (segment (start 128.905 55.88) (end 121.285 55.88) (width 0.254) (layer F.Cu) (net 34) (status 400000))
 (segment (start 106.68 73.66) (end 106.68 86.36) (width 0.254) (layer F.Cu) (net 34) (status 800000))
 (segment (start 111.125 69.215) (end 106.68 73.66) (width 0.254) (layer F.Cu) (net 34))
 (segment (start 114.935 69.215) (end 111.125 69.215) (width 0.254) (layer F.Cu) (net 34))
 (segment (start 118.11 66.04) (end 114.935 69.215) (width 0.254) (layer F.Cu) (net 34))
 (segment (start 118.11 59.055) (end 118.11 66.04) (width 0.254) (layer F.Cu) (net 34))
 (segment (start 121.285 55.88) (end 118.11 59.055) (width 0.254) (layer F.Cu) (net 34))
 (segment (start 128.905 58.42) (end 121.285 58.42) (width 0.254) (layer F.Cu) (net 35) (status 400000))
 (segment (start 122.555 86.36) (end 132.08 86.36) (width 0.254) (layer F.Cu) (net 35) (status 800000))
 (segment (start 118.745 82.55) (end 122.555 86.36) (width 0.254) (layer F.Cu) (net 35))
 (segment (start 118.745 60.96) (end 118.745 82.55) (width 0.254) (layer F.Cu) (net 35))
 (segment (start 121.285 58.42) (end 118.745 60.96) (width 0.254) (layer F.Cu) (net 35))
 (segment (start 128.905 60.96) (end 122.555 60.96) (width 0.254) (layer F.Cu) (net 36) (status 400000))
 (segment (start 154.94 85.09) (end 154.94 86.36) (width 0.254) (layer F.Cu) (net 36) (status 800000))
 (segment (start 153.035 83.185) (end 154.94 85.09) (width 0.254) (layer F.Cu) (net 36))
 (segment (start 123.19 83.185) (end 153.035 83.185) (width 0.254) (layer F.Cu) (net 36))
 (segment (start 120.015 80.01) (end 123.19 83.185) (width 0.254) (layer F.Cu) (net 36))
 (segment (start 120.015 63.5) (end 120.015 80.01) (width 0.254) (layer F.Cu) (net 36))
 (segment (start 122.555 60.96) (end 120.015 63.5) (width 0.254) (layer F.Cu) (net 36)))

